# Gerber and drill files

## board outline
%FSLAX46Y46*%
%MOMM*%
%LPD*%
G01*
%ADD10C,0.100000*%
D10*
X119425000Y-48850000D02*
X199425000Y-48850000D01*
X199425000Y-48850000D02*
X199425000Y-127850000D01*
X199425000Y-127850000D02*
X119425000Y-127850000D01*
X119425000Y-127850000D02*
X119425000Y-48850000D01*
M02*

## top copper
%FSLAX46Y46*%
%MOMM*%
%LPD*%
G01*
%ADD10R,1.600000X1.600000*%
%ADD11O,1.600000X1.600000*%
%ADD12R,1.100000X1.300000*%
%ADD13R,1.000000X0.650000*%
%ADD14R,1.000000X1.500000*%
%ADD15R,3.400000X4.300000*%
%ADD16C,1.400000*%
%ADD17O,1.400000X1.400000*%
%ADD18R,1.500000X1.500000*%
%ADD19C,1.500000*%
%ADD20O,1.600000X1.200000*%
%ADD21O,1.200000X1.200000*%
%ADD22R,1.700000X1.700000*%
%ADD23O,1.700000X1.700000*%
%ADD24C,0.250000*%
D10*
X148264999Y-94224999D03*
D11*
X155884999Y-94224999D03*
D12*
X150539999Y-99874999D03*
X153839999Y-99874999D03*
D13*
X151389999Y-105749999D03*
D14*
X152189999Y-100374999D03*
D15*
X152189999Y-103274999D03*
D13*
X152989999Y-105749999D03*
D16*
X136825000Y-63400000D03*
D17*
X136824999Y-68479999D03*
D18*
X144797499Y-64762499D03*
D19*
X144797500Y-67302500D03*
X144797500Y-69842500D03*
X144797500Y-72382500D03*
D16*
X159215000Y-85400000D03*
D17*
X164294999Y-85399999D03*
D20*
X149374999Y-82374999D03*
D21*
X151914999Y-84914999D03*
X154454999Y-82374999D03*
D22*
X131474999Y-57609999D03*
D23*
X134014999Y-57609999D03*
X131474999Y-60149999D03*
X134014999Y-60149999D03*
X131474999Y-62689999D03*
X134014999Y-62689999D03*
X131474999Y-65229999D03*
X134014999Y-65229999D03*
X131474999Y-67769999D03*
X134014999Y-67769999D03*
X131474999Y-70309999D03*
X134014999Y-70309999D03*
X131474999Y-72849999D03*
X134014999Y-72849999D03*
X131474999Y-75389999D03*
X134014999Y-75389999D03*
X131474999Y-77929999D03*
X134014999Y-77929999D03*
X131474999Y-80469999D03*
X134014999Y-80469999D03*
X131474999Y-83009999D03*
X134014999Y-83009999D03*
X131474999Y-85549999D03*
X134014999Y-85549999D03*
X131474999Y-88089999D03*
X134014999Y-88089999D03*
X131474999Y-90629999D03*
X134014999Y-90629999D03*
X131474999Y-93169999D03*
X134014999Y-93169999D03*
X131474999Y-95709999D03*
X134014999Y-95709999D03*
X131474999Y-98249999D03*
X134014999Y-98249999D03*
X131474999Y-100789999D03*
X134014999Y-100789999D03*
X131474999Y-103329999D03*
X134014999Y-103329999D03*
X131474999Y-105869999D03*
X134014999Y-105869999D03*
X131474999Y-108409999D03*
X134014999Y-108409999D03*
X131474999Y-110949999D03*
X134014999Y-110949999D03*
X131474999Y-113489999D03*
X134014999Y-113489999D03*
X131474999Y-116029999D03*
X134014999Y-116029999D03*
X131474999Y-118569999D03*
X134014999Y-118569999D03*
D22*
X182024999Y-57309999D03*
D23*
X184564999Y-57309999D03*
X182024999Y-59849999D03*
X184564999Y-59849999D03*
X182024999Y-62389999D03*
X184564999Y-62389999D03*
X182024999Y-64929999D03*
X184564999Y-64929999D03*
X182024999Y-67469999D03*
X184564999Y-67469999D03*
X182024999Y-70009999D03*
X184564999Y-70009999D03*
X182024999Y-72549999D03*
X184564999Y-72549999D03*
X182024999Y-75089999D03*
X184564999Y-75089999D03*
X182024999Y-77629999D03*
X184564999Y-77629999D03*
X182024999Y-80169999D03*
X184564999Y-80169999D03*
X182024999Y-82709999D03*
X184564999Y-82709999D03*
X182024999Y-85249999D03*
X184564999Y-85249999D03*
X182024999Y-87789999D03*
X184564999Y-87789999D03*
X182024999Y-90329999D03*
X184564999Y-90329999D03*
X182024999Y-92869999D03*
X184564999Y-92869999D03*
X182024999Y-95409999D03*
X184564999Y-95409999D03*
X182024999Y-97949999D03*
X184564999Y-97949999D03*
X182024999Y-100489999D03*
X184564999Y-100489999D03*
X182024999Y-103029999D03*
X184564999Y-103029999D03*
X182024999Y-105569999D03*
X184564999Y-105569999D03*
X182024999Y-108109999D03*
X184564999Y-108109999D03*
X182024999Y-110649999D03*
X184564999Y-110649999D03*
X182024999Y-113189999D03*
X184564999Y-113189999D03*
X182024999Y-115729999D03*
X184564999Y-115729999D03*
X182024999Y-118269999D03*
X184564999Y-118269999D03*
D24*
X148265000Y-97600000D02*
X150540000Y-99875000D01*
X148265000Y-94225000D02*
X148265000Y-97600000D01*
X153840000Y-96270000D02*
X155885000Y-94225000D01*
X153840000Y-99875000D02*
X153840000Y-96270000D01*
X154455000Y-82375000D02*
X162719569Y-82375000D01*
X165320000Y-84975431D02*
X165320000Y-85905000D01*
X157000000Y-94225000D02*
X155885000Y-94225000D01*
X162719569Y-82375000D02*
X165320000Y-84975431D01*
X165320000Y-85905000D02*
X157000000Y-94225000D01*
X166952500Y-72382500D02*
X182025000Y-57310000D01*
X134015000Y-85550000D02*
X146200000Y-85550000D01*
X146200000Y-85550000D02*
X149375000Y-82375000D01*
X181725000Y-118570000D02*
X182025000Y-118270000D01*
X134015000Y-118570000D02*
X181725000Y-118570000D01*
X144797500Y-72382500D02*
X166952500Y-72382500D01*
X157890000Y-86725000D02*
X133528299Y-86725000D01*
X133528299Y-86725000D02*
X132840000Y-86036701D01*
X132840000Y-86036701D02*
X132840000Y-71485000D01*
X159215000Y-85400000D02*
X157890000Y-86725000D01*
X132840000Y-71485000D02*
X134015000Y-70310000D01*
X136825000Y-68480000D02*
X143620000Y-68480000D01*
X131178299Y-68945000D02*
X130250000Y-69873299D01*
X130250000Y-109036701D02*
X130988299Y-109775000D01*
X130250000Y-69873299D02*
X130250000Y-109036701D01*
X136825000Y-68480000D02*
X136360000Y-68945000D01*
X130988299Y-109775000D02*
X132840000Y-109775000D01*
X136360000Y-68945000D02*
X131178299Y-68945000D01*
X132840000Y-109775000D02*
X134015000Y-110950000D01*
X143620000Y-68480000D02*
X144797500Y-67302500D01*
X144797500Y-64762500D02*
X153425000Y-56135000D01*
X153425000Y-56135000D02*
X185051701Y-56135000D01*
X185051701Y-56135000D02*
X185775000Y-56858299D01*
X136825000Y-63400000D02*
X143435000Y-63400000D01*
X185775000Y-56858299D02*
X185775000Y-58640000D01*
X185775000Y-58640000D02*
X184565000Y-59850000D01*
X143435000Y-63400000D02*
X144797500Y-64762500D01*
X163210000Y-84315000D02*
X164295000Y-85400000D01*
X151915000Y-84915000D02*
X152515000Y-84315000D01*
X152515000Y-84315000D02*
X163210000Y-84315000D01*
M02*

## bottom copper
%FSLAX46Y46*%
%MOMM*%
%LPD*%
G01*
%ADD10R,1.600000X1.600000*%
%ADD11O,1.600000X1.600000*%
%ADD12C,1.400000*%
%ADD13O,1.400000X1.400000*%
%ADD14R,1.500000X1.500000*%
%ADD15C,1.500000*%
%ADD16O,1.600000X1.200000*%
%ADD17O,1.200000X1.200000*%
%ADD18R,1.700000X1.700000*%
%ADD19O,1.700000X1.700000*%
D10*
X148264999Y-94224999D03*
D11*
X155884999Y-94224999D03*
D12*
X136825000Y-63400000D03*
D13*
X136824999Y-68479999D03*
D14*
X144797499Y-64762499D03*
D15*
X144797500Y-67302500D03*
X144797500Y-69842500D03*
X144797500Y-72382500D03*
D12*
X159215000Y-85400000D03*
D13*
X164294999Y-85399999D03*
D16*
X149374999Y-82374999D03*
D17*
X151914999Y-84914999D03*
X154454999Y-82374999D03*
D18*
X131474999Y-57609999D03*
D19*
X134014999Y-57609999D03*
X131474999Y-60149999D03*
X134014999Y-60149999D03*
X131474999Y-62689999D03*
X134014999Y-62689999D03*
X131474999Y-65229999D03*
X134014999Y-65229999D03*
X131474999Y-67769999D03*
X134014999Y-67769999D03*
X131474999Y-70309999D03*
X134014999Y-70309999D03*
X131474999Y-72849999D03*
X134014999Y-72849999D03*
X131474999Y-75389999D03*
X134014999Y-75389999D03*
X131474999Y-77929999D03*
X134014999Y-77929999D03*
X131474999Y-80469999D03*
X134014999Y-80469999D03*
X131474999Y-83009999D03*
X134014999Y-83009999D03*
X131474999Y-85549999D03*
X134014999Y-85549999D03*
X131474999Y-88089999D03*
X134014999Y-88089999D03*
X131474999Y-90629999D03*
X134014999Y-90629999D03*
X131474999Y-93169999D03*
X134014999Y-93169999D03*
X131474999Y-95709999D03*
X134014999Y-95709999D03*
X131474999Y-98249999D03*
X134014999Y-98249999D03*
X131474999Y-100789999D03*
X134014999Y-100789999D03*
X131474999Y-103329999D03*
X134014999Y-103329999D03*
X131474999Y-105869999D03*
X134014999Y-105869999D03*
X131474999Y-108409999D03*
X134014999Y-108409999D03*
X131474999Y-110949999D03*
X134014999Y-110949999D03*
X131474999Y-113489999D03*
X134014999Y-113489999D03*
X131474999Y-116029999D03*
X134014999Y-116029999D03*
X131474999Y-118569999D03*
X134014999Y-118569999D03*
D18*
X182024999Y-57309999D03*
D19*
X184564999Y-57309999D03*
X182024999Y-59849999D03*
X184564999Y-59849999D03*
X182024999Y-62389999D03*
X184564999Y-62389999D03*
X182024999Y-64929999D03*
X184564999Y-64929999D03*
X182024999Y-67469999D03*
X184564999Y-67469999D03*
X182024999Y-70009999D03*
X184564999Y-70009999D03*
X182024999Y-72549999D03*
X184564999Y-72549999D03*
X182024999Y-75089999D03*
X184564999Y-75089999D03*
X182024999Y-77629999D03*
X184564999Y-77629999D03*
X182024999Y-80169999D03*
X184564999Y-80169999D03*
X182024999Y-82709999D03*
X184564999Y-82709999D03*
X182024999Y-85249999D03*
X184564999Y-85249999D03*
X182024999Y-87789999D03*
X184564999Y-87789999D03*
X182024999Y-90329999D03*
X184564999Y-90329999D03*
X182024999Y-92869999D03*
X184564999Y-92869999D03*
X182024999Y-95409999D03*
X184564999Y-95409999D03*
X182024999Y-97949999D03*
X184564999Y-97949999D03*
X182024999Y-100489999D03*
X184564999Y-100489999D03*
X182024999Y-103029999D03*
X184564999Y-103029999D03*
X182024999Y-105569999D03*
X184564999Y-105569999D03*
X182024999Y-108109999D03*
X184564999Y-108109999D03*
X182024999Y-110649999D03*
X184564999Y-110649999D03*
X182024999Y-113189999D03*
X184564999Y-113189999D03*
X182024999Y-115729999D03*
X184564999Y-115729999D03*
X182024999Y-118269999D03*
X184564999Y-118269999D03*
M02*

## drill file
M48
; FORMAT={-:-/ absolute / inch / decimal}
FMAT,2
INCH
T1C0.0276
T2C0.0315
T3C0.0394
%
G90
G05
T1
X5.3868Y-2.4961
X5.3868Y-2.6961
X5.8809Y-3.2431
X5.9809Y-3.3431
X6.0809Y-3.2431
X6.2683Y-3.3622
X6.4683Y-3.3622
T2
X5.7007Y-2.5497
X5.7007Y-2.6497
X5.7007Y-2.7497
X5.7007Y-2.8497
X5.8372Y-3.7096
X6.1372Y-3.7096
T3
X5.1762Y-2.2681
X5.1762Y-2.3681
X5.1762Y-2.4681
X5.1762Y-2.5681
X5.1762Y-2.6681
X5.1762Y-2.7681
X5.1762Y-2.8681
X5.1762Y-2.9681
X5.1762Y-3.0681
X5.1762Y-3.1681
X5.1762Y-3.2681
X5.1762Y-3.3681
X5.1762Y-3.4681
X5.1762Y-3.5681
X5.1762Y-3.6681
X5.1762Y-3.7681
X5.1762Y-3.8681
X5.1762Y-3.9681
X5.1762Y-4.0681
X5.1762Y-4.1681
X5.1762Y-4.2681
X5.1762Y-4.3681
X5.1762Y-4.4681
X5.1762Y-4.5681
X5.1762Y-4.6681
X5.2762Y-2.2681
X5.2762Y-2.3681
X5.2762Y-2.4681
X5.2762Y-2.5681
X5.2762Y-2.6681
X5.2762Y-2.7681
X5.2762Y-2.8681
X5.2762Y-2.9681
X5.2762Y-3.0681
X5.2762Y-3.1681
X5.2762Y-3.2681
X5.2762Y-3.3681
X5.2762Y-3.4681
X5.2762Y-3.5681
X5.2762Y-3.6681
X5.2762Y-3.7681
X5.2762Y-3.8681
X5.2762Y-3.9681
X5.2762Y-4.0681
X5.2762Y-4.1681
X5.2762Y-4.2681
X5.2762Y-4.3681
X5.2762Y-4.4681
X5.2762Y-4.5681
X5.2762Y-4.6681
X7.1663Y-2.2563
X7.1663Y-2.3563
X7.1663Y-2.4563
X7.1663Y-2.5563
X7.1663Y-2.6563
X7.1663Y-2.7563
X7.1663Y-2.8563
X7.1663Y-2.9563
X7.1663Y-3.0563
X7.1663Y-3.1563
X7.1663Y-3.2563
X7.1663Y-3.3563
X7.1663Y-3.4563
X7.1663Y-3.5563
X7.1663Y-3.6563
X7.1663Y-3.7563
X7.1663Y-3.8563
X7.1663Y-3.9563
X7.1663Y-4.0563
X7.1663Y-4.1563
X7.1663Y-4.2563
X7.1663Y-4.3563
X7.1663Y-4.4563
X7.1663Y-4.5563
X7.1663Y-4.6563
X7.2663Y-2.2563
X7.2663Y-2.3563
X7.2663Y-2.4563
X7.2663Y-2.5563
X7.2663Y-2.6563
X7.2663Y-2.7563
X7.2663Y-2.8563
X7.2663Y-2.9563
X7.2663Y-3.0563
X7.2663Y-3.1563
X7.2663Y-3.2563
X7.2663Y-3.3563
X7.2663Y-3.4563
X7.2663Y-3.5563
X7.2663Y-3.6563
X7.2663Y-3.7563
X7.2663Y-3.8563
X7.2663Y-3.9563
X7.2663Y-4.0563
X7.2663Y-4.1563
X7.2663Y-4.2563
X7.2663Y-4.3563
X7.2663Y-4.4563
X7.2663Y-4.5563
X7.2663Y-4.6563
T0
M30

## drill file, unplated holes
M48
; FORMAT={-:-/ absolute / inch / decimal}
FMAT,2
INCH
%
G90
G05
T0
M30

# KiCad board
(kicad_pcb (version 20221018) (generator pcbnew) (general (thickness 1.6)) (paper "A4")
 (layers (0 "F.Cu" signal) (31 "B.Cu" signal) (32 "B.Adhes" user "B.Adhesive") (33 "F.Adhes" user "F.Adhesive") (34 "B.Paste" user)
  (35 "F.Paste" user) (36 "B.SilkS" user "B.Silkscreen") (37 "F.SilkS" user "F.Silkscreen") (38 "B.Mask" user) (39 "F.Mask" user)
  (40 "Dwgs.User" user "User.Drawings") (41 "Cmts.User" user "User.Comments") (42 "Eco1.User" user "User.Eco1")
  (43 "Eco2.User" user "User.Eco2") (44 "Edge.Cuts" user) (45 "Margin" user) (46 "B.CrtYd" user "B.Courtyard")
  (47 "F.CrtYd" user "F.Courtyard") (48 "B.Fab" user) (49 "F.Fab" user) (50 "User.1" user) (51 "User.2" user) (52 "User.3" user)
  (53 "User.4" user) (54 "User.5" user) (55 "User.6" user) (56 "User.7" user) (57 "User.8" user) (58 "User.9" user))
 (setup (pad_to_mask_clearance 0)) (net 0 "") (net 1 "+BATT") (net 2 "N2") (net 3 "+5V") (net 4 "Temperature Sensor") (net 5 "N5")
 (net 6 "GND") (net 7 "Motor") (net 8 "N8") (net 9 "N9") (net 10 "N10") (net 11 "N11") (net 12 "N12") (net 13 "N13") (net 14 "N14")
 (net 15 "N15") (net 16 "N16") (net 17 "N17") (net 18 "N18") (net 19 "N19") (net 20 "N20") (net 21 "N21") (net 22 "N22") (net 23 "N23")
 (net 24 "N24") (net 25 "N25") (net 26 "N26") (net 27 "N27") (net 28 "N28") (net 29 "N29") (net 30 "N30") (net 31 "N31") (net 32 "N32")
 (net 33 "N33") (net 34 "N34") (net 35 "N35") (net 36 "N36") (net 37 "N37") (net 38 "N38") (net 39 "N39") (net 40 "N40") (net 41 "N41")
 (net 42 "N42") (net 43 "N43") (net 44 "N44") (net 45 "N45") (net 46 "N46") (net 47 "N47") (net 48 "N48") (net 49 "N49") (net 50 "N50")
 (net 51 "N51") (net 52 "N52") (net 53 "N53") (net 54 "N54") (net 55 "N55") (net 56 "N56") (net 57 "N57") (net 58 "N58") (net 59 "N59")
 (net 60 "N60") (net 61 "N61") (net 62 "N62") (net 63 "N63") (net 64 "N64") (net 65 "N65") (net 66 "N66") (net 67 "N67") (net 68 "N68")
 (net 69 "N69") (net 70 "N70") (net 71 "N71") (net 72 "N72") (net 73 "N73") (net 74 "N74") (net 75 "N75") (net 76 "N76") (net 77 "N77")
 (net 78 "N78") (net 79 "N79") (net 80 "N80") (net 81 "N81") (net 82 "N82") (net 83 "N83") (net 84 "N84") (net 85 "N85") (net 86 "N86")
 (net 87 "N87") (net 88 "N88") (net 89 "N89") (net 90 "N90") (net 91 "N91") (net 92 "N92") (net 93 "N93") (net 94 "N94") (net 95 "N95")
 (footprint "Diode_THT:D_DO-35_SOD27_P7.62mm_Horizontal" (layer "F.Cu") (at 148.265 94.225)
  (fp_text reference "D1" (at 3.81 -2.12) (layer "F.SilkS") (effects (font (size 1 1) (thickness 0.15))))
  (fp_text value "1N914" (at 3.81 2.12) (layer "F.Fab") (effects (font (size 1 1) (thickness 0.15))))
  (pad "1" thru_hole rect (at 0 0) (size 1.6 1.6) (drill 0.8) (layers "*.Cu" "*.Mask") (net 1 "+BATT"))
  (pad "2" thru_hole oval (at 7.62 0) (size 1.6 1.6) (drill 0.8) (layers "*.Cu" "*.Mask") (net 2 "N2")))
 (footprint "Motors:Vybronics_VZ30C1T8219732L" (layer "F.Cu") (at 152.19 104.225)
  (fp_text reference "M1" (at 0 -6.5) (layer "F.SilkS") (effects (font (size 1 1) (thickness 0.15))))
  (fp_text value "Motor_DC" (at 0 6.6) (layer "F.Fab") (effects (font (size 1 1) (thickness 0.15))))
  (pad "" smd rect (at -0.85 -2.315 270) (size 1.07 1.4) (layers "F.Paste"))
  (pad "" smd rect (at -0.85 -0.905 270) (size 1.07 1.4) (layers "F.Paste"))
  (pad "" smd rect (at -0.85 0.505 270) (size 1.07 1.4) (layers "F.Paste"))
  (pad "" smd rect (at 0.85 -2.315 270) (size 1.07 1.4) (layers "F.Paste"))
  (pad "" smd rect (at 0.85 -0.905 270) (size 1.07 1.4) (layers "F.Paste"))
  (pad "" smd rect (at 0.85 0.505 270) (size 1.07 1.4) (layers "F.Paste"))
  (pad "1" smd rect (at -1.65 -4.35 270) (size 1.3 1.1) (layers "F.Cu" "F.Paste" "F.Mask") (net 1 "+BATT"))
  (pad "2" smd rect (at 1.65 -4.35 270) (size 1.3 1.1) (layers "F.Cu" "F.Paste" "F.Mask") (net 2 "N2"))
  (pad "SH" smd rect (at -0.8 1.525) (size 1 0.65) (layers "F.Cu" "F.Paste" "F.Mask"))
  (pad "SH" smd rect (at 0 -3.85 270) (size 1.5 1) (layers "F.Cu" "F.Paste" "F.Mask"))
  (pad "SH" smd rect (at 0 -0.95 270) (size 4.3 3.4) (layers "F.Cu" "F.Mask"))
  (pad "SH" smd rect (at 0.8 1.525) (size 1 0.65) (layers "F.Cu" "F.Paste" "F.Mask")))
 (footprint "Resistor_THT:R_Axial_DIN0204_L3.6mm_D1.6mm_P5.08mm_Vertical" (layer "F.Cu") (at 136.825 63.4 -90)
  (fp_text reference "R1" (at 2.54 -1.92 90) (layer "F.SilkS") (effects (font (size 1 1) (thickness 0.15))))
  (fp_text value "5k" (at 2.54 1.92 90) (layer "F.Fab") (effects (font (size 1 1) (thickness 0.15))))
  (pad "1" thru_hole circle (at 0 0 270) (size 1.4 1.4) (drill 0.7) (layers "*.Cu" "*.Mask") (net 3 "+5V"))
  (pad "2" thru_hole oval (at 5.08 0 270) (size 1.4 1.4) (drill 0.7) (layers "*.Cu" "*.Mask") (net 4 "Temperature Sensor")))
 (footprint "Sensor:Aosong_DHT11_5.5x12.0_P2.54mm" (layer "F.Cu") (at 144.7975 64.7625)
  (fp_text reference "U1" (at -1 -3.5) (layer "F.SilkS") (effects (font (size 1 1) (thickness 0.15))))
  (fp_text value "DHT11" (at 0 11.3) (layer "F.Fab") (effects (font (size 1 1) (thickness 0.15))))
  (pad "1" thru_hole rect (at 0 0) (size 1.5 1.5) (drill 0.8) (layers "*.Cu" "*.Mask") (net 3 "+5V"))
  (pad "2" thru_hole circle (at 0 2.54) (size 1.5 1.5) (drill 0.8) (layers "*.Cu" "*.Mask") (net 4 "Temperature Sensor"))
  (pad "3" thru_hole circle (at 0 5.08) (size 1.5 1.5) (drill 0.8) (layers "*.Cu" "*.Mask") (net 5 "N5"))
  (pad "4" thru_hole circle (at 0 7.62) (size 1.5 1.5) (drill 0.8) (layers "*.Cu" "*.Mask") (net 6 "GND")))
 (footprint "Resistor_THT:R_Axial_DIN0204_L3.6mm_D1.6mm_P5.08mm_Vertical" (layer "F.Cu") (at 159.215 85.4)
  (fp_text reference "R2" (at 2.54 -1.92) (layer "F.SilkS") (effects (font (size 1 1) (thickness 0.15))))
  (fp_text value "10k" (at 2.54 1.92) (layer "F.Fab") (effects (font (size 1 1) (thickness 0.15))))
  (pad "1" thru_hole circle (at 0 0) (size 1.4 1.4) (drill 0.7) (layers "*.Cu" "*.Mask") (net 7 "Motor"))
  (pad "2" thru_hole oval (at 5.08 0) (size 1.4 1.4) (drill 0.7) (layers "*.Cu" "*.Mask") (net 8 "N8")))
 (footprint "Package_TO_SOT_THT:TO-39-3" (layer "F.Cu") (at 149.375 82.375)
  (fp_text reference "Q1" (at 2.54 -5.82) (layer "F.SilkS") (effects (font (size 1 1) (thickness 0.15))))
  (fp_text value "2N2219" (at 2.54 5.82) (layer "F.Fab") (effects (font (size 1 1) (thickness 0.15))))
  (pad "1" thru_hole oval (at 0 0) (size 1.6 1.2) (drill 0.7) (layers "*.Cu" "*.Mask") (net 6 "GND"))
  (pad "2" thru_hole oval (at 2.54 2.54) (size 1.2 1.2) (drill 0.7) (layers "*.Cu" "*.Mask") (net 8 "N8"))
  (pad "3" thru_hole oval (at 5.08 0) (size 1.2 1.2) (drill 0.7) (layers "*.Cu" "*.Mask") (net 2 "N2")))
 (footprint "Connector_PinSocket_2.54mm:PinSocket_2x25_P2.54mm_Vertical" (layer "B.Cu") (at 131.475 57.61 180)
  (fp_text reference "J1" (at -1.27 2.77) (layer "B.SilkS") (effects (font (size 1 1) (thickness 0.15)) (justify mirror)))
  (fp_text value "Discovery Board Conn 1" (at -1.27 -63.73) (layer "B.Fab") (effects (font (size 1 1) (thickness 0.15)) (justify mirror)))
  (pad "1" thru_hole rect (at 0 0 180) (size 1.7 1.7) (drill 1) (layers "*.Cu" "*.Mask") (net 6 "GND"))
  (pad "2" thru_hole oval (at -2.54 0 180) (size 1.7 1.7) (drill 1) (layers "*.Cu" "*.Mask") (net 6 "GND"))
  (pad "3" thru_hole oval (at 0 -2.54 180) (size 1.7 1.7) (drill 1) (layers "*.Cu" "*.Mask") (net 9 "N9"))
  (pad "4" thru_hole oval (at -2.54 -2.54 180) (size 1.7 1.7) (drill 1) (layers "*.Cu" "*.Mask") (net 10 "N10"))
  (pad "5" thru_hole oval (at 0 -5.08 180) (size 1.7 1.7) (drill 1) (layers "*.Cu" "*.Mask") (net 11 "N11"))
  (pad "6" thru_hole oval (at -2.54 -5.08 180) (size 1.7 1.7) (drill 1) (layers "*.Cu" "*.Mask") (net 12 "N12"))
  (pad "7" thru_hole oval (at 0 -7.62 180) (size 1.7 1.7) (drill 1) (layers "*.Cu" "*.Mask") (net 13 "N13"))
  (pad "8" thru_hole oval (at -2.54 -7.62 180) (size 1.7 1.7) (drill 1) (layers "*.Cu" "*.Mask") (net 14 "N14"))
  (pad "9" thru_hole oval (at 0 -10.16 180) (size 1.7 1.7) (drill 1) (layers "*.Cu" "*.Mask") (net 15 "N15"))
  (pad "10" thru_hole oval (at -2.54 -10.16 180) (size 1.7 1.7) (drill 1) (layers "*.Cu" "*.Mask") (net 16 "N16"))
  (pad "11" thru_hole oval (at 0 -12.7 180) (size 1.7 1.7) (drill 1) (layers "*.Cu" "*.Mask") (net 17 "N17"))
  (pad "12" thru_hole oval (at -2.54 -12.7 180) (size 1.7 1.7) (drill 1) (layers "*.Cu" "*.Mask") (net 7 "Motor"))
  (pad "13" thru_hole oval (at 0 -15.24 180) (size 1.7 1.7) (drill 1) (layers "*.Cu" "*.Mask") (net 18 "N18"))
  (pad "14" thru_hole oval (at -2.54 -15.24 180) (size 1.7 1.7) (drill 1) (layers "*.Cu" "*.Mask") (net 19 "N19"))
  (pad "15" thru_hole oval (at 0 -17.78 180) (size 1.7 1.7) (drill 1) (layers "*.Cu" "*.Mask") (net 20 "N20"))
  (pad "16" thru_hole oval (at -2.54 -17.78 180) (size 1.7 1.7) (drill 1) (layers "*.Cu" "*.Mask") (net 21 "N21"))
  (pad "17" thru_hole oval (at 0 -20.32 180) (size 1.7 1.7) (drill 1) (layers "*.Cu" "*.Mask") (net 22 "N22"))
  (pad "18" thru_hole oval (at -2.54 -20.32 180) (size 1.7 1.7) (drill 1) (layers "*.Cu" "*.Mask") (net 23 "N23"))
  (pad "19" thru_hole oval (at 0 -22.86 180) (size 1.7 1.7) (drill 1) (layers "*.Cu" "*.Mask") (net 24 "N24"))
  (pad "20" thru_hole oval (at -2.54 -22.86 180) (size 1.7 1.7) (drill 1) (layers "*.Cu" "*.Mask") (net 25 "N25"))
  (pad "21" thru_hole oval (at 0 -25.4 180) (size 1.7 1.7) (drill 1) (layers "*.Cu" "*.Mask") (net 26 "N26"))
  (pad "22" thru_hole oval (at -2.54 -25.4 180) (size 1.7 1.7) (drill 1) (layers "*.Cu" "*.Mask") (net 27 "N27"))
  (pad "23" thru_hole oval (at 0 -27.94 180) (size 1.7 1.7) (drill 1) (layers "*.Cu" "*.Mask") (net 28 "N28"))
  (pad "24" thru_hole oval (at -2.54 -27.94 180) (size 1.7 1.7) (drill 1) (layers "*.Cu" "*.Mask") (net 6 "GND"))
  (pad "25" thru_hole oval (at 0 -30.48 180) (size 1.7 1.7) (drill 1) (layers "*.Cu" "*.Mask") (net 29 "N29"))
  (pad "26" thru_hole oval (at -2.54 -30.48 180) (size 1.7 1.7) (drill 1) (layers "*.Cu" "*.Mask") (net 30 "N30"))
  (pad "27" thru_hole oval (at 0 -33.02 180) (size 1.7 1.7) (drill 1) (layers "*.Cu" "*.Mask") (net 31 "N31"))
  (pad "28" thru_hole oval (at -2.54 -33.02 180) (size 1.7 1.7) (drill 1) (layers "*.Cu" "*.Mask") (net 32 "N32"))
  (pad "29" thru_hole oval (at 0 -35.56 180) (size 1.7 1.7) (drill 1) (layers "*.Cu" "*.Mask") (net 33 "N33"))
  (pad "30" thru_hole oval (at -2.54 -35.56 180) (size 1.7 1.7) (drill 1) (layers "*.Cu" "*.Mask") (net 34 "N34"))
  (pad "31" thru_hole oval (at 0 -38.1 180) (size 1.7 1.7) (drill 1) (layers "*.Cu" "*.Mask") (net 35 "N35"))
  (pad "32" thru_hole oval (at -2.54 -38.1 180) (size 1.7 1.7) (drill 1) (layers "*.Cu" "*.Mask") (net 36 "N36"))
  (pad "33" thru_hole oval (at 0 -40.64 180) (size 1.7 1.7) (drill 1) (layers "*.Cu" "*.Mask") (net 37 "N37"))
  (pad "34" thru_hole oval (at -2.54 -40.64 180) (size 1.7 1.7) (drill 1) (layers "*.Cu" "*.Mask") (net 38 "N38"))
  (pad "35" thru_hole oval (at 0 -43.18 180) (size 1.7 1.7) (drill 1) (layers "*.Cu" "*.Mask") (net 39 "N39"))
  (pad "36" thru_hole oval (at -2.54 -43.18 180) (size 1.7 1.7) (drill 1) (layers "*.Cu" "*.Mask") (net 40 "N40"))
  (pad "37" thru_hole oval (at 0 -45.72 180) (size 1.7 1.7) (drill 1) (layers "*.Cu" "*.Mask") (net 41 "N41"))
  (pad "38" thru_hole oval (at -2.54 -45.72 180) (size 1.7 1.7) (drill 1) (layers "*.Cu" "*.Mask") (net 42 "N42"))
  (pad "39" thru_hole oval (at 0 -48.26 180) (size 1.7 1.7) (drill 1) (layers "*.Cu" "*.Mask") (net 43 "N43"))
  (pad "40" thru_hole oval (at -2.54 -48.26 180) (size 1.7 1.7) (drill 1) (layers "*.Cu" "*.Mask") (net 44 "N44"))
  (pad "41" thru_hole oval (at 0 -50.8 180) (size 1.7 1.7) (drill 1) (layers "*.Cu" "*.Mask") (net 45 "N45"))
  (pad "42" thru_hole oval (at -2.54 -50.8 180) (size 1.7 1.7) (drill 1) (layers "*.Cu" "*.Mask") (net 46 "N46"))
  (pad "43" thru_hole oval (at 0 -53.34 180) (size 1.7 1.7) (drill 1) (layers "*.Cu" "*.Mask") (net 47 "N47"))
  (pad "44" thru_hole oval (at -2.54 -53.34 180) (size 1.7 1.7) (drill 1) (layers "*.Cu" "*.Mask") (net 4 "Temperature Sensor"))
  (pad "45" thru_hole oval (at 0 -55.88 180) (size 1.7 1.7) (drill 1) (layers "*.Cu" "*.Mask") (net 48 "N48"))
  (pad "46" thru_hole oval (at -2.54 -55.88 180) (size 1.7 1.7) (drill 1) (layers "*.Cu" "*.Mask") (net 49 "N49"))
  (pad "47" thru_hole oval (at 0 -58.42 180) (size 1.7 1.7) (drill 1) (layers "*.Cu" "*.Mask") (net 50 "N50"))
  (pad "48" thru_hole oval (at -2.54 -58.42 180) (size 1.7 1.7) (drill 1) (layers "*.Cu" "*.Mask") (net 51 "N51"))
  (pad "49" thru_hole oval (at 0 -60.96 180) (size 1.7 1.7) (drill 1) (layers "*.Cu" "*.Mask") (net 6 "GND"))
  (pad "50" thru_hole oval (at -2.54 -60.96 180) (size 1.7 1.7) (drill 1) (layers "*.Cu" "*.Mask") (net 6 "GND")))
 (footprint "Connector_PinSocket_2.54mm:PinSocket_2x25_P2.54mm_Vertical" (layer "B.Cu") (at 182.025 57.31 180)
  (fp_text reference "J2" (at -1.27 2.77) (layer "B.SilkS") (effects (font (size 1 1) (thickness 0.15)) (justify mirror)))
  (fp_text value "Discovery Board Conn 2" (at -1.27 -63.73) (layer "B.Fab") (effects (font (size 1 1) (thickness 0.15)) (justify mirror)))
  (pad "1" thru_hole rect (at 0 0 180) (size 1.7 1.7) (drill 1) (layers "*.Cu" "*.Mask") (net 6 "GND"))
  (pad "2" thru_hole oval (at -2.54 0 180) (size 1.7 1.7) (drill 1) (layers "*.Cu" "*.Mask") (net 6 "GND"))
  (pad "3" thru_hole oval (at 0 -2.54 180) (size 1.7 1.7) (drill 1) (layers "*.Cu" "*.Mask") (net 3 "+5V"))
  (pad "4" thru_hole oval (at -2.54 -2.54 180) (size 1.7 1.7) (drill 1) (layers "*.Cu" "*.Mask") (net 3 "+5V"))
  (pad "5" thru_hole oval (at 0 -5.08 180) (size 1.7 1.7) (drill 1) (layers "*.Cu" "*.Mask") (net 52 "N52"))
  (pad "6" thru_hole oval (at -2.54 -5.08 180) (size 1.7 1.7) (drill 1) (layers "*.Cu" "*.Mask") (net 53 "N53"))
  (pad "7" thru_hole oval (at 0 -7.62 180) (size 1.7 1.7) (drill 1) (layers "*.Cu" "*.Mask") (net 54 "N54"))
  (pad "8" thru_hole oval (at -2.54 -7.62 180) (size 1.7 1.7) (drill 1) (layers "*.Cu" "*.Mask") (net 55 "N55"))
  (pad "9" thru_hole oval (at 0 -10.16 180) (size 1.7 1.7) (drill 1) (layers "*.Cu" "*.Mask") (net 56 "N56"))
  (pad "10" thru_hole oval (at -2.54 -10.16 180) (size 1.7 1.7) (drill 1) (layers "*.Cu" "*.Mask") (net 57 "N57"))
  (pad "11" thru_hole oval (at 0 -12.7 180) (size 1.7 1.7) (drill 1) (layers "*.Cu" "*.Mask") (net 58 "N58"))
  (pad "12" thru_hole oval (at -2.54 -12.7 180) (size 1.7 1.7) (drill 1) (layers "*.Cu" "*.Mask") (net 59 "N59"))
  (pad "13" thru_hole oval (at 0 -15.24 180) (size 1.7 1.7) (drill 1) (layers "*.Cu" "*.Mask") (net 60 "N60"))
  (pad "14" thru_hole oval (at -2.54 -15.24 180) (size 1.7 1.7) (drill 1) (layers "*.Cu" "*.Mask") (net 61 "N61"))
  (pad "15" thru_hole oval (at 0 -17.78 180) (size 1.7 1.7) (drill 1) (layers "*.Cu" "*.Mask") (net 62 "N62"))
  (pad "16" thru_hole oval (at -2.54 -17.78 180) (size 1.7 1.7) (drill 1) (layers "*.Cu" "*.Mask") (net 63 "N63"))
  (pad "17" thru_hole oval (at 0 -20.32 180) (size 1.7 1.7) (drill 1) (layers "*.Cu" "*.Mask") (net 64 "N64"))
  (pad "18" thru_hole oval (at -2.54 -20.32 180) (size 1.7 1.7) (drill 1) (layers "*.Cu" "*.Mask") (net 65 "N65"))
  (pad "19" thru_hole oval (at 0 -22.86 180) (size 1.7 1.7) (drill 1) (layers "*.Cu" "*.Mask") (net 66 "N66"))
  (pad "20" thru_hole oval (at -2.54 -22.86 180) (size 1.7 1.7) (drill 1) (layers "*.Cu" "*.Mask") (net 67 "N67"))
  (pad "21" thru_hole oval (at 0 -25.4 180) (size 1.7 1.7) (drill 1) (layers "*.Cu" "*.Mask") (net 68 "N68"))
  (pad "22" thru_hole oval (at -2.54 -25.4 180) (size 1.7 1.7) (drill 1) (layers "*.Cu" "*.Mask") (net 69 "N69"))
  (pad "23" thru_hole oval (at 0 -27.94 180) (size 1.7 1.7) (drill 1) (layers "*.Cu" "*.Mask") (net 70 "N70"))
  (pad "24" thru_hole oval (at -2.54 -27.94 180) (size 1.7 1.7) (drill 1) (layers "*.Cu" "*.Mask") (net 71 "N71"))
  (pad "25" thru_hole oval (at 0 -30.48 180) (size 1.7 1.7) (drill 1) (layers "*.Cu" "*.Mask") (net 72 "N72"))
  (pad "26" thru_hole oval (at -2.54 -30.48 180) (size 1.7 1.7) (drill 1) (layers "*.Cu" "*.Mask") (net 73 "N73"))
  (pad "27" thru_hole oval (at 0 -33.02 180) (size 1.7 1.7) (drill 1) (layers "*.Cu" "*.Mask") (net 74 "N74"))
  (pad "28" thru_hole oval (at -2.54 -33.02 180) (size 1.7 1.7) (drill 1) (layers "*.Cu" "*.Mask") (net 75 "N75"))
  (pad "29" thru_hole oval (at 0 -35.56 180) (size 1.7 1.7) (drill 1) (layers "*.Cu" "*.Mask") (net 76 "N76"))
  (pad "30" thru_hole oval (at -2.54 -35.56 180) (size 1.7 1.7) (drill 1) (layers "*.Cu" "*.Mask") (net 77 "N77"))
  (pad "31" thru_hole oval (at 0 -38.1 180) (size 1.7 1.7) (drill 1) (layers "*.Cu" "*.Mask") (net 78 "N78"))
  (pad "32" thru_hole oval (at -2.54 -38.1 180) (size 1.7 1.7) (drill 1) (layers "*.Cu" "*.Mask") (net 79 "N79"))
  (pad "33" thru_hole oval (at 0 -40.64 180) (size 1.7 1.7) (drill 1) (layers "*.Cu" "*.Mask") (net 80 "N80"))
  (pad "34" thru_hole oval (at -2.54 -40.64 180) (size 1.7 1.7) (drill 1) (layers "*.Cu" "*.Mask") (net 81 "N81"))
  (pad "35" thru_hole oval (at 0 -43.18 180) (size 1.7 1.7) (drill 1) (layers "*.Cu" "*.Mask") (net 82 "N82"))
  (pad "36" thru_hole oval (at -2.54 -43.18 180) (size 1.7 1.7) (drill 1) (layers "*.Cu" "*.Mask") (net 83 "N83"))
  (pad "37" thru_hole oval (at 0 -45.72 180) (size 1.7 1.7) (drill 1) (layers "*.Cu" "*.Mask") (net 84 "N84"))
  (pad "38" thru_hole oval (at -2.54 -45.72 180) (size 1.7 1.7) (drill 1) (layers "*.Cu" "*.Mask") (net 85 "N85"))
  (pad "39" thru_hole oval (at 0 -48.26 180) (size 1.7 1.7) (drill 1) (layers "*.Cu" "*.Mask") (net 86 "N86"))
  (pad "40" thru_hole oval (at -2.54 -48.26 180) (size 1.7 1.7) (drill 1) (layers "*.Cu" "*.Mask") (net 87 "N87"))
  (pad "41" thru_hole oval (at 0 -50.8 180) (size 1.7 1.7) (drill 1) (layers "*.Cu" "*.Mask") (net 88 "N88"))
  (pad "42" thru_hole oval (at -2.54 -50.8 180) (size 1.7 1.7) (drill 1) (layers "*.Cu" "*.Mask") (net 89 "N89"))
  (pad "43" thru_hole oval (at 0 -53.34 180) (size 1.7 1.7) (drill 1) (layers "*.Cu" "*.Mask") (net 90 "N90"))
  (pad "44" thru_hole oval (at -2.54 -53.34 180) (size 1.7 1.7) (drill 1) (layers "*.Cu" "*.Mask") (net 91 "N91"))
  (pad "45" thru_hole oval (at 0 -55.88 180) (size 1.7 1.7) (drill 1) (layers "*.Cu" "*.Mask") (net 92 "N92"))
  (pad "46" thru_hole oval (at -2.54 -55.88 180) (size 1.7 1.7) (drill 1) (layers "*.Cu" "*.Mask") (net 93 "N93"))
  (pad "47" thru_hole oval (at 0 -58.42 180) (size 1.7 1.7) (drill 1) (layers "*.Cu" "*.Mask") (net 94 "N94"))
  (pad "48" thru_hole oval (at -2.54 -58.42 180) (size 1.7 1.7) (drill 1) (layers "*.Cu" "*.Mask") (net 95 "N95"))
  (pad "49" thru_hole oval (at 0 -60.96 180) (size 1.7 1.7) (drill 1) (layers "*.Cu" "*.Mask") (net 6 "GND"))
  (pad "50" thru_hole oval (at -2.54 -60.96 180) (size 1.7 1.7) (drill 1) (layers "*.Cu" "*.Mask") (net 6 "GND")))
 (gr_rect (start 119.425 48.85) (end 199.425 127.85) (stroke (width 0.1) (type default)) (fill none) (layer "Edge.Cuts"))
 (segment (start 148.265 97.6) (end 150.54 99.875) (width 0.25) (layer "F.Cu") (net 1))
 (segment (start 148.265 94.225) (end 148.265 97.6) (width 0.25) (layer "F.Cu") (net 1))
 (segment (start 153.84 96.27) (end 155.885 94.225) (width 0.25) (layer "F.Cu") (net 2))
 (segment (start 153.84 99.875) (end 153.84 96.27) (width 0.25) (layer "F.Cu") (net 2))
 (segment (start 154.455 82.375) (end 162.719569 82.375) (width 0.25) (layer "F.Cu") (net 2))
 (segment (start 165.32 84.975431) (end 165.32 85.905) (width 0.25) (layer "F.Cu") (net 2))
 (segment (start 157 94.225) (end 155.885 94.225) (width 0.25) (layer "F.Cu") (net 2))
 (segment (start 162.719569 82.375) (end 165.32 84.975431) (width 0.25) (layer "F.Cu") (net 2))
 (segment (start 165.32 85.905) (end 157 94.225) (width 0.25) (layer "F.Cu") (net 2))
 (segment (start 166.9525 72.3825) (end 182.025 57.31) (width 0.25) (layer "F.Cu") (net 6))
 (segment (start 134.015 85.55) (end 146.2 85.55) (width 0.25) (layer "F.Cu") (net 6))
 (segment (start 146.2 85.55) (end 149.375 82.375) (width 0.25) (layer "F.Cu") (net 6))
 (segment (start 181.725 118.57) (end 182.025 118.27) (width 0.25) (layer "F.Cu") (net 6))
 (segment (start 134.015 118.57) (end 181.725 118.57) (width 0.25) (layer "F.Cu") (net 6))
 (segment (start 144.7975 72.3825) (end 166.9525 72.3825) (width 0.25) (layer "F.Cu") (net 6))
 (segment (start 157.89 86.725) (end 133.528299 86.725) (width 0.25) (layer "F.Cu") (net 7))
 (segment (start 133.528299 86.725) (end 132.84 86.036701) (width 0.25) (layer "F.Cu") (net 7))
 (segment (start 132.84 86.036701) (end 132.84 71.485) (width 0.25) (layer "F.Cu") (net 7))
 (segment (start 159.215 85.4) (end 157.89 86.725) (width 0.25) (layer "F.Cu") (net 7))
 (segment (start 132.84 71.485) (end 134.015 70.31) (width 0.25) (layer "F.Cu") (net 7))
 (segment (start 136.825 68.48) (end 143.62 68.48) (width 0.25) (layer "F.Cu") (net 4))
 (segment (start 131.178299 68.945) (end 130.25 69.873299) (width 0.25) (layer "F.Cu") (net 4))
 (segment (start 130.25 109.036701) (end 130.988299 109.775) (width 0.25) (layer "F.Cu") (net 4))
 (segment (start 130.25 69.873299) (end 130.25 109.036701) (width 0.25) (layer "F.Cu") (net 4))
 (segment (start 136.825 68.48) (end 136.36 68.945) (width 0.25) (layer "F.Cu") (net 4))
 (segment (start 130.988299 109.775) (end 132.84 109.775) (width 0.25) (layer "F.Cu") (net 4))
 (segment (start 136.36 68.945) (end 131.178299 68.945) (width 0.25) (layer "F.Cu") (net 4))
 (segment (start 132.84 109.775) (end 134.015 110.95) (width 0.25) (layer "F.Cu") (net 4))
 (segment (start 143.62 68.48) (end 144.7975 67.3025) (width 0.25) (layer "F.Cu") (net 4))
 (segment (start 144.7975 64.7625) (end 153.425 56.135) (width 0.25) (layer "F.Cu") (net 3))
 (segment (start 153.425 56.135) (end 185.051701 56.135) (width 0.25) (layer "F.Cu") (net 3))
 (segment (start 185.051701 56.135) (end 185.775 56.858299) (width 0.25) (layer "F.Cu") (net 3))
 (segment (start 136.825 63.4) (end 143.435 63.4) (width 0.25) (layer "F.Cu") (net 3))
 (segment (start 185.775 56.858299) (end 185.775 58.64) (width 0.25) (layer "F.Cu") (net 3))
 (segment (start 185.775 58.64) (end 184.565 59.85) (width 0.25) (layer "F.Cu") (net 3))
 (segment (start 143.435 63.4) (end 144.7975 64.7625) (width 0.25) (layer "F.Cu") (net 3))
 (segment (start 163.21 84.315) (end 164.295 85.4) (width 0.25) (layer "F.Cu") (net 8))
 (segment (start 151.915 84.915) (end 152.515 84.315) (width 0.25) (layer "F.Cu") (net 8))
 (segment (start 152.515 84.315) (end 163.21 84.315) (width 0.25) (layer "F.Cu") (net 8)))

